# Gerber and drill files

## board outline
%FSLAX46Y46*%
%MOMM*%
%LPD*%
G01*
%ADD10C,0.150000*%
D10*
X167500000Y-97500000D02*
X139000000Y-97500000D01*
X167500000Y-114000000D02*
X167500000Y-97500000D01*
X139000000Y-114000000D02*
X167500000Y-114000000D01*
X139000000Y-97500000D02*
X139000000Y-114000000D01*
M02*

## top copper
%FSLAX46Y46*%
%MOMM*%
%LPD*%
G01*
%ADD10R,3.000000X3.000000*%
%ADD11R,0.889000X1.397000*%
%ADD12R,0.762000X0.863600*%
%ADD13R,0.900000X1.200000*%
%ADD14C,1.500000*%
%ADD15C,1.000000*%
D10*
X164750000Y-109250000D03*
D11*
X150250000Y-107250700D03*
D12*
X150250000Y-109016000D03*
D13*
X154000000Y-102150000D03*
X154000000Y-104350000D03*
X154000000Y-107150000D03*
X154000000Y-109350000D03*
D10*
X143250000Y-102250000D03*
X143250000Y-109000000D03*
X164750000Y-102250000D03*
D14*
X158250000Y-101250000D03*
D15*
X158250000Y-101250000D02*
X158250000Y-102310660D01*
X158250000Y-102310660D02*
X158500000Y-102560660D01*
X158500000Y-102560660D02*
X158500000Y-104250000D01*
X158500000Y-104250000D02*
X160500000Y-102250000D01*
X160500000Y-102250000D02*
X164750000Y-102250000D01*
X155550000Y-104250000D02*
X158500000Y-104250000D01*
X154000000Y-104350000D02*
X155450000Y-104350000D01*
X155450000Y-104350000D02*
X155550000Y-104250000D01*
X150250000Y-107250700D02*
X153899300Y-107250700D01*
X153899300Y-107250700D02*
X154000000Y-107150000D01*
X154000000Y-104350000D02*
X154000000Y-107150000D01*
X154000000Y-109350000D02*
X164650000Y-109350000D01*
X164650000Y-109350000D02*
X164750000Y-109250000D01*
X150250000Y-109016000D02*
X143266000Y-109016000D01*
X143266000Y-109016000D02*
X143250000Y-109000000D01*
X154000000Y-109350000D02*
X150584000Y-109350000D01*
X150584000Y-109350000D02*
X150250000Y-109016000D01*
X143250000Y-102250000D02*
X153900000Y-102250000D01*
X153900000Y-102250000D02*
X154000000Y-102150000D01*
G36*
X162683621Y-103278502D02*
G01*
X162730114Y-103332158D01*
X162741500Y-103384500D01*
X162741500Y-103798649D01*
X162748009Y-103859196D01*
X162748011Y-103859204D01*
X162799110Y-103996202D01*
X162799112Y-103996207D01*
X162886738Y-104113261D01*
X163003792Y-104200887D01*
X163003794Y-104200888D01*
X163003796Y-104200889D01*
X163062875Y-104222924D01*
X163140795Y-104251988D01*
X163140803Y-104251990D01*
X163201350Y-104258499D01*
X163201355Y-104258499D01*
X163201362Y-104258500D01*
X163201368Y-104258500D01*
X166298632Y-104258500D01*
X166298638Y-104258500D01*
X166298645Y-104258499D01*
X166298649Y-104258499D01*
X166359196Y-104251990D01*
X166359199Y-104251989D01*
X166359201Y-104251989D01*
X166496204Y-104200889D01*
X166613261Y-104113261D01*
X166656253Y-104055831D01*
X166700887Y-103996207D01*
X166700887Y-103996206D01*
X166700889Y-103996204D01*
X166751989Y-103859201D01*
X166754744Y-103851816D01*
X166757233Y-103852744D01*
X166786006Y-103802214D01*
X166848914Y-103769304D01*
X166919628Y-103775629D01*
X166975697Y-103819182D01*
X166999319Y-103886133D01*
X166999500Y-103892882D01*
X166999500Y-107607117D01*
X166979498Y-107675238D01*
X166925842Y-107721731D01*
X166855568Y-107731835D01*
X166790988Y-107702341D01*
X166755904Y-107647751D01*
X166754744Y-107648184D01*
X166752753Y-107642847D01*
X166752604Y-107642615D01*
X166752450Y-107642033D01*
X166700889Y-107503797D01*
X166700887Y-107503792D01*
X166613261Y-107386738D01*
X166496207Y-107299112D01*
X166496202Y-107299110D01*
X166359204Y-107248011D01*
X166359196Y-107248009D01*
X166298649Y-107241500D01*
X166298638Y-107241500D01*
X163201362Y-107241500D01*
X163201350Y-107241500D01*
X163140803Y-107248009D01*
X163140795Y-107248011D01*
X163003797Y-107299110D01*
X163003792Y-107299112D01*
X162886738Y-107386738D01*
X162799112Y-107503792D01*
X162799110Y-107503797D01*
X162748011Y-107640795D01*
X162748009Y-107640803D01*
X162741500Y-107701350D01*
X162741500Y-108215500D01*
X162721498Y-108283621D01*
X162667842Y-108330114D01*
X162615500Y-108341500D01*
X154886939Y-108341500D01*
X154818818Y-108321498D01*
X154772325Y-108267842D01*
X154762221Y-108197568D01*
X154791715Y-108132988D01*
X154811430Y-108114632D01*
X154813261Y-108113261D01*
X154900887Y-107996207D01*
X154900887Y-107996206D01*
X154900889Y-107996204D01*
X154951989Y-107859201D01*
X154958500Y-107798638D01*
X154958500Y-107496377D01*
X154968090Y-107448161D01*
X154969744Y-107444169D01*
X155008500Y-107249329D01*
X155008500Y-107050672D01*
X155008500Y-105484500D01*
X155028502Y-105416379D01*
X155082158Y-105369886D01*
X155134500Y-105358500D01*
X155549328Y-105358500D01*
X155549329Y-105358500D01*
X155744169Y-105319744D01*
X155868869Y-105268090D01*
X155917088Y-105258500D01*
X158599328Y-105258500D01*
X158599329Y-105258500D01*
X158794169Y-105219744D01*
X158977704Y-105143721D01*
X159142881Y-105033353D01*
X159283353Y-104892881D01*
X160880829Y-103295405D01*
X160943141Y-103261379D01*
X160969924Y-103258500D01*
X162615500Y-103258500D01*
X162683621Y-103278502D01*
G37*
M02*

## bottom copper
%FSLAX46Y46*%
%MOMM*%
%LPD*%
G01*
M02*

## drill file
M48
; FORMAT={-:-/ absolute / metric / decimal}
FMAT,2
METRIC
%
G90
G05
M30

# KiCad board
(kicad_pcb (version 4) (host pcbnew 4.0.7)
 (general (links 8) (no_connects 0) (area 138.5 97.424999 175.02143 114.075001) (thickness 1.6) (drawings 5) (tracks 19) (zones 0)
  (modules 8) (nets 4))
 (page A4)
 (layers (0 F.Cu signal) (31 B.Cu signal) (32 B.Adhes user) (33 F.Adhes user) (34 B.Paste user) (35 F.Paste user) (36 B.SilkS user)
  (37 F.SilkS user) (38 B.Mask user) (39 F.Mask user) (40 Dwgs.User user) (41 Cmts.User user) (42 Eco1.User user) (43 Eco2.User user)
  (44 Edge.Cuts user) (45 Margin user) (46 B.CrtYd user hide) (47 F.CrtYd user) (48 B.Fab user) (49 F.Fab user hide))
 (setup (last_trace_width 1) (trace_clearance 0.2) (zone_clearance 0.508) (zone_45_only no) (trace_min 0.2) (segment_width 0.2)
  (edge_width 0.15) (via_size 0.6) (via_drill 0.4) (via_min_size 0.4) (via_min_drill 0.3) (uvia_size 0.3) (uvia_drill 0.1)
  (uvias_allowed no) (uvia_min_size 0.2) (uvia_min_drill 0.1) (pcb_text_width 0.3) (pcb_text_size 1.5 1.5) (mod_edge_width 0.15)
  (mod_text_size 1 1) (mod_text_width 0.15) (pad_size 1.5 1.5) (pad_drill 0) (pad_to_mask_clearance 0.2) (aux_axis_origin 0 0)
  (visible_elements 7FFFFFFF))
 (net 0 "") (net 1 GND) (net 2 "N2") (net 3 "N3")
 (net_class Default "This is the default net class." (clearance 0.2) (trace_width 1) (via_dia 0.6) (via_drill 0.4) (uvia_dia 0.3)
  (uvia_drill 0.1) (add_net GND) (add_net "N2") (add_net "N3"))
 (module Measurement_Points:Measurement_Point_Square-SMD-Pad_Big (layer F.Cu) (at 164.75 109.25)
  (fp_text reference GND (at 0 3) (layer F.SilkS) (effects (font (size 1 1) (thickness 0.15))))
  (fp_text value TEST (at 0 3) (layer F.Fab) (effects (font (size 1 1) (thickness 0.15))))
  (pad 1 smd rect (at 0 0) (size 3 3) (layers F.Cu F.Mask) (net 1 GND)))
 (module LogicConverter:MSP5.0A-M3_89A (layer F.Cu) (at 150.25 108 270)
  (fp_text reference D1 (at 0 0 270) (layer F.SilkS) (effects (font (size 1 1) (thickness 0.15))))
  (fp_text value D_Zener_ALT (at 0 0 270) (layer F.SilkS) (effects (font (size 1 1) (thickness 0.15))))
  (pad 1 smd rect (at -0.7493 0 270) (size 1.397 0.889) (layers F.Cu F.Paste F.Mask) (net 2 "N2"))
  (pad 2 smd rect (at 1.016 0 270) (size 0.8636 0.762) (layers F.Cu F.Paste F.Mask) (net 1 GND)))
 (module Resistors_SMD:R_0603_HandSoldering (layer F.Cu) (at 154 103.25 270)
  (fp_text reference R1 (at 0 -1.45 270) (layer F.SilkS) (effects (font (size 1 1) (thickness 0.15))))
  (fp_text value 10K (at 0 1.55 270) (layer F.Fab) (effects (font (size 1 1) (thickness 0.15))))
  (pad 1 smd rect (at -1.1 0 270) (size 1.2 0.9) (layers F.Cu F.Paste F.Mask) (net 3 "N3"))
  (pad 2 smd rect (at 1.1 0 270) (size 1.2 0.9) (layers F.Cu F.Paste F.Mask) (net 2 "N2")))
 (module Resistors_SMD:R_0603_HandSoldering (layer F.Cu) (at 154 108.25 270)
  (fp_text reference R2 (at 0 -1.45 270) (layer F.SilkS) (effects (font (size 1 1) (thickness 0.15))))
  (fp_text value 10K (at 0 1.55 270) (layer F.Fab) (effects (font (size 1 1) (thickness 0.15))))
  (pad 1 smd rect (at -1.1 0 270) (size 1.2 0.9) (layers F.Cu F.Paste F.Mask) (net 2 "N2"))
  (pad 2 smd rect (at 1.1 0 270) (size 1.2 0.9) (layers F.Cu F.Paste F.Mask) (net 1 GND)))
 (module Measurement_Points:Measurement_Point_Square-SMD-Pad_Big (layer F.Cu) (at 143.25 102.25)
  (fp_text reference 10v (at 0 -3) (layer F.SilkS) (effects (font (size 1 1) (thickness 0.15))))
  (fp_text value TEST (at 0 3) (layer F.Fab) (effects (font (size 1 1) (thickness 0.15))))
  (pad 1 smd rect (at 0 0) (size 3 3) (layers F.Cu F.Mask) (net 3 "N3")))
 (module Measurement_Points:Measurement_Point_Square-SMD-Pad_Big (layer F.Cu) (at 143.25 109)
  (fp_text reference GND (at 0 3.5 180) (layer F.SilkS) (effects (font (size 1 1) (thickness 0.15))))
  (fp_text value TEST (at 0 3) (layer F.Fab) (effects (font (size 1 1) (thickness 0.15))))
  (pad 1 smd rect (at 0 0) (size 3 3) (layers F.Cu F.Mask) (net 1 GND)))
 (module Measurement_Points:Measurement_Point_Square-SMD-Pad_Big (layer F.Cu) (at 164.75 102.25)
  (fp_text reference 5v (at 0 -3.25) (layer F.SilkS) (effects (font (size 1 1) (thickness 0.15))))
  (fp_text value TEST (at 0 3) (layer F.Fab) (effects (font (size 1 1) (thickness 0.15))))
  (pad 1 smd rect (at 0 0) (size 3 3) (layers F.Cu F.Mask) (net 2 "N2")))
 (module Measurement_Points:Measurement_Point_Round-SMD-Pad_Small (layer F.Cu) (at 158.25 101.25)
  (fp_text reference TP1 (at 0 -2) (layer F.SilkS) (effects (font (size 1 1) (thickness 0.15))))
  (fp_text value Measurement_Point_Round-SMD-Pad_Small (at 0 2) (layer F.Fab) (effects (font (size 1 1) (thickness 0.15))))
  (pad 1 smd circle (at 0 0) (size 1.5 1.5) (layers F.Cu F.Mask) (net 2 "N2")))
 (gr_line (start 167.5 97.5) (end 139 97.5) (layer Edge.Cuts) (width 0.15))
 (gr_line (start 167.5 114) (end 167.5 97.5) (layer Edge.Cuts) (width 0.15))
 (gr_line (start 139 114) (end 167.5 114) (layer Edge.Cuts) (width 0.15))
 (gr_line (start 139 97.5) (end 139 114) (layer Edge.Cuts) (width 0.15))
 (segment (start 158.25 101.25) (end 158.25 102.31066) (width 1) (layer F.Cu) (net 2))
 (segment (start 158.25 102.31066) (end 158.5 102.56066) (width 1) (layer F.Cu) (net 2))
 (segment (start 158.5 102.56066) (end 158.5 104.25) (width 1) (layer F.Cu) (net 2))
 (segment (start 158.5 104.25) (end 160.5 102.25) (width 1) (layer F.Cu) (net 2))
 (segment (start 160.5 102.25) (end 164.75 102.25) (width 1) (layer F.Cu) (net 2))
 (segment (start 155.55 104.25) (end 158.5 104.25) (width 1) (layer F.Cu) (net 2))
 (segment (start 154 104.35) (end 155.45 104.35) (width 1) (layer F.Cu) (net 2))
 (segment (start 155.45 104.35) (end 155.55 104.25) (width 1) (layer F.Cu) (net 2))
 (segment (start 150.25 107.2507) (end 153.8993 107.2507) (width 1) (layer F.Cu) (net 2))
 (segment (start 153.8993 107.2507) (end 154 107.15) (width 1) (layer F.Cu) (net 2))
 (segment (start 154 104.35) (end 154 107.15) (width 1) (layer F.Cu) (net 2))
 (segment (start 154 109.35) (end 164.65 109.35) (width 1) (layer F.Cu) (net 1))
 (segment (start 164.65 109.35) (end 164.75 109.25) (width 1) (layer F.Cu) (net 1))
 (segment (start 150.25 109.016) (end 143.266 109.016) (width 1) (layer F.Cu) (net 1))
 (segment (start 143.266 109.016) (end 143.25 109) (width 1) (layer F.Cu) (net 1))
 (segment (start 154 109.35) (end 150.584 109.35) (width 1) (layer F.Cu) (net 1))
 (segment (start 150.584 109.35) (end 150.25 109.016) (width 1) (layer F.Cu) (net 1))
 (segment (start 143.25 102.25) (end 153.9 102.25) (width 1) (layer F.Cu) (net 3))
 (segment (start 153.9 102.25) (end 154 102.15) (width 1) (layer F.Cu) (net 3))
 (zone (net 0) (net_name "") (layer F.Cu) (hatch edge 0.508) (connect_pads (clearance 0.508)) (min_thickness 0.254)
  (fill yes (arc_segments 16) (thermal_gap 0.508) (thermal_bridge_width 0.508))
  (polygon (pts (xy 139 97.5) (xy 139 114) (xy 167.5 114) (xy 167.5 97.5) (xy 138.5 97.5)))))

